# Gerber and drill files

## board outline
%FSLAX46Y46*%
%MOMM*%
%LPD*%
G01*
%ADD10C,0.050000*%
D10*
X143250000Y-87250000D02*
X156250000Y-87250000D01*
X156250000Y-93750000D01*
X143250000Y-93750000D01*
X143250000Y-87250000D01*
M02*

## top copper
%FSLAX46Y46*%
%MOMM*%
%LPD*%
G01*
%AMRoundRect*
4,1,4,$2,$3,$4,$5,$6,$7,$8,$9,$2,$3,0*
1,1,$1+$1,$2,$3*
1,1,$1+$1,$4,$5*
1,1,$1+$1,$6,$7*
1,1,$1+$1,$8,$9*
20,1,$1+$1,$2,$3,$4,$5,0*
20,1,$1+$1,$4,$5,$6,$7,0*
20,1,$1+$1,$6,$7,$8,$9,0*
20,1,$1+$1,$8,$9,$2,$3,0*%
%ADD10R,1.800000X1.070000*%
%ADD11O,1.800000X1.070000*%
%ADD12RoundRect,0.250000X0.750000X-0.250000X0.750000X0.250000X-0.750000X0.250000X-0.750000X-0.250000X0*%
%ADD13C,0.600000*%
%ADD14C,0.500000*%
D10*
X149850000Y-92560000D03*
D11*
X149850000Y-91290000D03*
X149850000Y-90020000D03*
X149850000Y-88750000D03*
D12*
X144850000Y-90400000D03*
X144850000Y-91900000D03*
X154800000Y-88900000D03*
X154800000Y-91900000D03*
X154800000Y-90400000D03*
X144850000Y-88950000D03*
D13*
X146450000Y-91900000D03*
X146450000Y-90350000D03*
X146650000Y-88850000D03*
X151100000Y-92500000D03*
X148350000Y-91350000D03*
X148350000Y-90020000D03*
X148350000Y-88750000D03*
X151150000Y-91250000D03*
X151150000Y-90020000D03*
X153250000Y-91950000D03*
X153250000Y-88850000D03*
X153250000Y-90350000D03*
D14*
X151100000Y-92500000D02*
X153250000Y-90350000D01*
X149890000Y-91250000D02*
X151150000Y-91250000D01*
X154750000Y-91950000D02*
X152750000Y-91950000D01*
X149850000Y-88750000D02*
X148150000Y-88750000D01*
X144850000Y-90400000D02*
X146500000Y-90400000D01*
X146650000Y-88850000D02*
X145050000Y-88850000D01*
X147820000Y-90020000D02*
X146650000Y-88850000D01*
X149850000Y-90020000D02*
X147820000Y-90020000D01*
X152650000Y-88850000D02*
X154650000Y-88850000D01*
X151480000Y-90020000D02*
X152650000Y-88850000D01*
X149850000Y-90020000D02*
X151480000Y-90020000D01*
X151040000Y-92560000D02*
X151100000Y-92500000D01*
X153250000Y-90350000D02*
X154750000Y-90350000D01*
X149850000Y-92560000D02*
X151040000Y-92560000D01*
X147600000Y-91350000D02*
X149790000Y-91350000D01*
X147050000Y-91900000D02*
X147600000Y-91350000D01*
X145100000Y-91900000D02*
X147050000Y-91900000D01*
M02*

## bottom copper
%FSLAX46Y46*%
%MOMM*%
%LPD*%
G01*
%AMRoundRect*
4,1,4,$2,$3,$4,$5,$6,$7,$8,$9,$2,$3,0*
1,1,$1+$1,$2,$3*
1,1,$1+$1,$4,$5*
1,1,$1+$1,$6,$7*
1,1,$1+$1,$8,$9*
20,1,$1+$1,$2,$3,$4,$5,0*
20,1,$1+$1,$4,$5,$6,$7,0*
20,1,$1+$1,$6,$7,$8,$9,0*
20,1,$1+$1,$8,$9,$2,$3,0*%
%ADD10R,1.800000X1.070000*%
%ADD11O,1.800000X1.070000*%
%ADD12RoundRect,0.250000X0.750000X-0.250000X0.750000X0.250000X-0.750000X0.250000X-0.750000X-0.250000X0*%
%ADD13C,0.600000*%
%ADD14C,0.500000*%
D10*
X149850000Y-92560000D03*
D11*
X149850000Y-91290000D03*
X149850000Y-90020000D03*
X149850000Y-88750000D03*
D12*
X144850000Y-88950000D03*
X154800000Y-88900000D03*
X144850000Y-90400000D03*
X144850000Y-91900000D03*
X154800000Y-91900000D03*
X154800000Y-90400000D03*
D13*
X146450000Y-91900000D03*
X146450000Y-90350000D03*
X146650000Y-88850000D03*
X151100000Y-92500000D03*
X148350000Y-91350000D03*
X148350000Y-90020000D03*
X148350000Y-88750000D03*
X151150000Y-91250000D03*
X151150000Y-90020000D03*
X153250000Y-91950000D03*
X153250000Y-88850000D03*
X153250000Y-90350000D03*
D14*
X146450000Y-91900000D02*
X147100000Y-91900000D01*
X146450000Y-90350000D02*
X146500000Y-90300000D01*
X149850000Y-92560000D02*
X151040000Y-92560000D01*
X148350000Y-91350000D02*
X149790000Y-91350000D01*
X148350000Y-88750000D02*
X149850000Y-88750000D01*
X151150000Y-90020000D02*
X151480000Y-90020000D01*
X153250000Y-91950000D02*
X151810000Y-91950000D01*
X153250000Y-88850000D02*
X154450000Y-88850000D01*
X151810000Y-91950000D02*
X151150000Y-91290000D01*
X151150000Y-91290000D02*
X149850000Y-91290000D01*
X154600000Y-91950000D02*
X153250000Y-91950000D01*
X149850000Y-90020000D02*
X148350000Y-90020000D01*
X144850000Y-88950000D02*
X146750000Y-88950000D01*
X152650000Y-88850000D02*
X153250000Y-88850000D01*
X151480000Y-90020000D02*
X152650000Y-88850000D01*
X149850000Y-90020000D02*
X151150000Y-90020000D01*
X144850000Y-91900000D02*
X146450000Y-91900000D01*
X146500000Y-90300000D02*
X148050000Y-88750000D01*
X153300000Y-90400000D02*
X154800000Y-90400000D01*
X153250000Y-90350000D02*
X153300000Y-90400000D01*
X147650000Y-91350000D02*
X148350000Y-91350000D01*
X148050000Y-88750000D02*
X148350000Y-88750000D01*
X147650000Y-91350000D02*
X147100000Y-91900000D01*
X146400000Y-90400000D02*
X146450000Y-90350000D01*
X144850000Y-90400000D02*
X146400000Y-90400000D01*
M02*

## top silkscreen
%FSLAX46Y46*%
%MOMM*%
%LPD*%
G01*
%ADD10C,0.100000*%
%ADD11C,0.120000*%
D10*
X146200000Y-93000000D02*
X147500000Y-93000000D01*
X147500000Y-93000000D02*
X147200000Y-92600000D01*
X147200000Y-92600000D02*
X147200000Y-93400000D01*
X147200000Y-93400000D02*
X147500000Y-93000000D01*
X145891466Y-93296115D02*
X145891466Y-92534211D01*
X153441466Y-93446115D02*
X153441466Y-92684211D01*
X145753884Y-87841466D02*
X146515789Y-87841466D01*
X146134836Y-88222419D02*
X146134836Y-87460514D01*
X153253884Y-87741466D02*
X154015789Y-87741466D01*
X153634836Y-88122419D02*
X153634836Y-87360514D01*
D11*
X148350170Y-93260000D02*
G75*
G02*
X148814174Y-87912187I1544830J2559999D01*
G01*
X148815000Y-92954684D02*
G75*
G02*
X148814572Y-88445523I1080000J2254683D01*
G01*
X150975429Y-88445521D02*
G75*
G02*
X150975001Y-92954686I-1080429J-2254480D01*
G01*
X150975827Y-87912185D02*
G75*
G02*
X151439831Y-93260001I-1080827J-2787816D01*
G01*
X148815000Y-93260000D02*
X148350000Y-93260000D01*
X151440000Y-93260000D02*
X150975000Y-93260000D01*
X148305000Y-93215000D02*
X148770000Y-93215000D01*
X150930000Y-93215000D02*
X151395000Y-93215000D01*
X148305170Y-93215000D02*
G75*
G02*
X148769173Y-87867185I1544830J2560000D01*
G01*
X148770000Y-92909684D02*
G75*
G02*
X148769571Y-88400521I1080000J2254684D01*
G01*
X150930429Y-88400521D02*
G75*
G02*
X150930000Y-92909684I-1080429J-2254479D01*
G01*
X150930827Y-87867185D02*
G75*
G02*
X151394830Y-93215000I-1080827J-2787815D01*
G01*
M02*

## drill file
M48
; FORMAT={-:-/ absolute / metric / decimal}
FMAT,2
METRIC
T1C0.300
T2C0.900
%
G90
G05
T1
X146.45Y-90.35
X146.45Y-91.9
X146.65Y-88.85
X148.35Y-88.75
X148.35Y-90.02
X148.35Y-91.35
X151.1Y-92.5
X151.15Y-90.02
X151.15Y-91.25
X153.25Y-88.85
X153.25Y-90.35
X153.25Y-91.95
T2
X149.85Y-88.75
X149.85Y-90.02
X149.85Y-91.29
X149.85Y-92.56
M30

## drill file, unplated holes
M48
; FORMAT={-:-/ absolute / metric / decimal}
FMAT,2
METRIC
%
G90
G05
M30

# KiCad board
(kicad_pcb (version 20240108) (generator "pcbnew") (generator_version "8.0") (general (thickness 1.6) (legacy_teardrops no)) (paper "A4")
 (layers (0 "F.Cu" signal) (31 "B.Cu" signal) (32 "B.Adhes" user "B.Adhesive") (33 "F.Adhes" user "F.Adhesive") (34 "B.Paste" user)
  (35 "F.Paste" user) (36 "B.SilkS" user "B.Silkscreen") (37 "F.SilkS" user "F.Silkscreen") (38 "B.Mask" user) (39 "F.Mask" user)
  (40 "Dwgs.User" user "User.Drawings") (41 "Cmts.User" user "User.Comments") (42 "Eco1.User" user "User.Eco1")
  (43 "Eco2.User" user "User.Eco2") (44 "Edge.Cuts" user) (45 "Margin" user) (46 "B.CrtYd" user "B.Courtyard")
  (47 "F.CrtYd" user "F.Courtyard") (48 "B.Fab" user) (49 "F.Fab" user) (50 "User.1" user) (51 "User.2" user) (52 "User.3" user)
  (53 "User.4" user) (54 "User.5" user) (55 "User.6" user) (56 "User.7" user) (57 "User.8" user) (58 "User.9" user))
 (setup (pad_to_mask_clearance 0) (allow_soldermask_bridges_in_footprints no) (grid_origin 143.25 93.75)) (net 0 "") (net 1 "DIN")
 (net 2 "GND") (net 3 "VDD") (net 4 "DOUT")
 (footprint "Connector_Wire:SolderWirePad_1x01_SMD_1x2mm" (layer "F.Cu") (at 144.85 90.4 90)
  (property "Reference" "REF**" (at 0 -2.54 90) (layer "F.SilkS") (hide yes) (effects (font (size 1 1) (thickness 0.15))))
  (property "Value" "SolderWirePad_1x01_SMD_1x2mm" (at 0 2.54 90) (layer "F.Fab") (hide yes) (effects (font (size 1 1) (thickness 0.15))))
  (pad "1" smd roundrect (at 0 0 90) (size 1 2) (layers "F.Cu" "F.Paste" "F.Mask") (roundrect_rratio 0.25) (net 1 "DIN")))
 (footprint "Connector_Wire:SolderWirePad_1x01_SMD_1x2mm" (layer "F.Cu") (at 144.85 91.9 90)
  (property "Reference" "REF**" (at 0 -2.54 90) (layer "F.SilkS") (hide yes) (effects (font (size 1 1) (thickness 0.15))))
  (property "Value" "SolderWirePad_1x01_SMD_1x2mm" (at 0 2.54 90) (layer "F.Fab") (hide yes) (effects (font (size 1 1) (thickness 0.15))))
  (pad "1" smd roundrect (at 0 0 90) (size 1 2) (layers "F.Cu" "F.Paste" "F.Mask") (roundrect_rratio 0.25) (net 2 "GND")))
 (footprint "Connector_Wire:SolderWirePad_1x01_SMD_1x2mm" (layer "F.Cu") (at 154.8 88.9 90)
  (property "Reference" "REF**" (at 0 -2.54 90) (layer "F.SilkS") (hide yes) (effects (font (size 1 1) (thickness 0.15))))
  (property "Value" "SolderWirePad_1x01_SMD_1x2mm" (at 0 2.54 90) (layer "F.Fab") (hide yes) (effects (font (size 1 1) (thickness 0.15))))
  (pad "1" smd roundrect (at 0 0 90) (size 1 2) (layers "F.Cu" "F.Paste" "F.Mask") (roundrect_rratio 0.25) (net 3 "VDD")))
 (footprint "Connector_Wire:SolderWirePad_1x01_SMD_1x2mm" (layer "F.Cu") (at 154.8 91.9 90)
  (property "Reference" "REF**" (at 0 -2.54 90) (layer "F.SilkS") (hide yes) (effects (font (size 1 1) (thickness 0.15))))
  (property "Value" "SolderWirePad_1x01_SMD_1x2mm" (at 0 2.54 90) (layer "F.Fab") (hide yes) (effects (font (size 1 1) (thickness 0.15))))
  (pad "1" smd roundrect (at 0 0 90) (size 1 2) (layers "F.Cu" "F.Paste" "F.Mask") (roundrect_rratio 0.25) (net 2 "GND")))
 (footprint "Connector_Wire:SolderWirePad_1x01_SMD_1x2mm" (layer "F.Cu") (at 154.8 90.4 90)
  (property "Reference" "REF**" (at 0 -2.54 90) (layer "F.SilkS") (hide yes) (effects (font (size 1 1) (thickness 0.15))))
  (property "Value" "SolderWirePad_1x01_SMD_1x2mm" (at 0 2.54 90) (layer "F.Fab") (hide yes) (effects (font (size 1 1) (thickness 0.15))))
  (pad "1" smd roundrect (at 0 0 90) (size 1 2) (layers "F.Cu" "F.Paste" "F.Mask") (roundrect_rratio 0.25) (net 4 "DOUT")))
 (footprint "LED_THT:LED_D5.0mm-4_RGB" (layer "F.Cu") (at 149.85 92.56 90)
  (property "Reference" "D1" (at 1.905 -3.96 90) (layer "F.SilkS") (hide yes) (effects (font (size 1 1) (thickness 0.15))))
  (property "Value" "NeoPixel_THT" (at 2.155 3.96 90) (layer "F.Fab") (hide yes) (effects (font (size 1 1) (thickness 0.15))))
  (fp_line (start -0.655 -1.545) (end -0.655 -1.08) (stroke (width 0.12) (type solid)) (layer "F.SilkS"))
  (fp_line (start -0.7 -1.035) (end -0.7 -1.5) (stroke (width 0.12) (type solid)) (layer "F.SilkS"))
  (fp_line (start -0.655 1.08) (end -0.655 1.545) (stroke (width 0.12) (type solid)) (layer "F.SilkS"))
  (fp_line (start -0.7 1.59) (end -0.7 1.125) (stroke (width 0.12) (type solid)) (layer "F.SilkS"))
  (fp_arc (start -0.655 -1.54483) (mid 2.163456 -2.978809) (end 4.692815 -1.080827) (stroke (width 0.12) (type solid)) (layer "F.SilkS"))
  (fp_arc (start -0.7 -1.49983) (mid 2.118456 -2.933808) (end 4.647815 -1.035827) (stroke (width 0.12) (type solid)) (layer "F.SilkS"))
  (fp_arc (start -0.349684 -1.08) (mid 1.904762 -2.5) (end 4.159479 -1.080429) (stroke (width 0.12) (type solid)) (layer "F.SilkS"))
  (fp_arc (start -0.394684 -1.035) (mid 1.859762 -2.454999) (end 4.114479 -1.035429) (stroke (width 0.12) (type solid)) (layer "F.SilkS"))
  (fp_arc (start 4.159479 1.080429) (mid 1.904762 2.5) (end -0.349684 1.08) (stroke (width 0.12) (type solid)) (layer "F.SilkS"))
  (fp_arc (start 4.692815 1.080827) (mid 2.163456 2.978808) (end -0.655 1.54483) (stroke (width 0.12) (type solid)) (layer "F.SilkS"))
  (fp_arc (start 4.114479 1.125429) (mid 1.859762 2.545001) (end -0.394684 1.125) (stroke (width 0.12) (type solid)) (layer "F.SilkS"))
  (fp_arc (start 4.647815 1.125827) (mid 2.118456 3.023809) (end -0.7 1.58983) (stroke (width 0.12) (type solid)) (layer "F.SilkS"))
  (pad "1" thru_hole rect (at 0 0 90) (size 1.07 1.8) (drill 0.9) (layers "*.Cu" "*.Mask") (remove_unused_layers no) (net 4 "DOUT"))
  (pad "2" thru_hole oval (at 1.27 0 90) (size 1.07 1.8) (drill 0.9) (layers "*.Cu" "*.Mask") (remove_unused_layers no) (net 2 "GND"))
  (pad "3" thru_hole oval (at 2.54 0 90) (size 1.07 1.8) (drill 0.9) (layers "*.Cu" "*.Mask") (remove_unused_layers no) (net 3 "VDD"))
  (pad "4" thru_hole oval (at 3.81 0 90) (size 1.07 1.8) (drill 0.9) (layers "*.Cu" "*.Mask") (remove_unused_layers no) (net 1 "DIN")))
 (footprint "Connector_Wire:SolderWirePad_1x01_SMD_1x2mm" (layer "F.Cu") (at 144.85 88.95 90)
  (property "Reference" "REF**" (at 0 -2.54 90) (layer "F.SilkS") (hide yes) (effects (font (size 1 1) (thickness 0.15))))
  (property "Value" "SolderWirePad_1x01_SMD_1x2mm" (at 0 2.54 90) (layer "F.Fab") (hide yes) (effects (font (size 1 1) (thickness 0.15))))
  (pad "1" smd roundrect (at 0 0 90) (size 1 2) (layers "F.Cu" "F.Paste" "F.Mask") (roundrect_rratio 0.25) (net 3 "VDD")))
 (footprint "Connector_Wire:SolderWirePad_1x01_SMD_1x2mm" (layer "B.Cu") (at 154.8 90.4 90)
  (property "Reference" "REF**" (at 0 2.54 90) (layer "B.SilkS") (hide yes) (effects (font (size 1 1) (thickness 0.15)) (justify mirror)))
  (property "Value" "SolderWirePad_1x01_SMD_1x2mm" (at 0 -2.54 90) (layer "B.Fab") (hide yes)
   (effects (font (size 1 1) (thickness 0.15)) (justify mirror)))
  (pad "1" smd roundrect (at 0 0 90) (size 1 2) (layers "B.Cu" "B.Paste" "B.Mask") (roundrect_rratio 0.25) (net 4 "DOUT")))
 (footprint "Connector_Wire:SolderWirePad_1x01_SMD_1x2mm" (layer "B.Cu") (at 144.85 88.95 90)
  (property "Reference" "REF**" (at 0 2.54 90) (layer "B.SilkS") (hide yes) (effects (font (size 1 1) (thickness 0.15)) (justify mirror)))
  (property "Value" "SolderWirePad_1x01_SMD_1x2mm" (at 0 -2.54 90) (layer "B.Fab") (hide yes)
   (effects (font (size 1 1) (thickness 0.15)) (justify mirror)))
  (pad "1" smd roundrect (at 0 0 90) (size 1 2) (layers "B.Cu" "B.Paste" "B.Mask") (roundrect_rratio 0.25) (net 3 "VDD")))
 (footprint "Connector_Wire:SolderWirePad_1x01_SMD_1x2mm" (layer "B.Cu") (at 154.8 88.9 90)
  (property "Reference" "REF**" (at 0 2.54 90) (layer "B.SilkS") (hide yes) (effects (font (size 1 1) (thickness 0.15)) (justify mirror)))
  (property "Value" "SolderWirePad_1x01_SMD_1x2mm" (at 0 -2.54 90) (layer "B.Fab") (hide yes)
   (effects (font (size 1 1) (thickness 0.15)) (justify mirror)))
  (pad "1" smd roundrect (at 0 0 90) (size 1 2) (layers "B.Cu" "B.Paste" "B.Mask") (roundrect_rratio 0.25) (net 3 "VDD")))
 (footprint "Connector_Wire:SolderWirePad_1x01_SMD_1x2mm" (layer "B.Cu") (at 144.85 90.4 90)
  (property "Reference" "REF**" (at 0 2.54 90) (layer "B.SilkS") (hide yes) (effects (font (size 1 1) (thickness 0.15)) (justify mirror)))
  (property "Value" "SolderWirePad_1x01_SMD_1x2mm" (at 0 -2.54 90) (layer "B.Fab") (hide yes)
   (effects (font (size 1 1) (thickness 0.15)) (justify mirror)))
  (pad "1" smd roundrect (at 0 0 90) (size 1 2) (layers "B.Cu" "B.Paste" "B.Mask") (roundrect_rratio 0.25) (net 1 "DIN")))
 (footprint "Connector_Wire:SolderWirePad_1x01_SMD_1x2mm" (layer "B.Cu") (at 144.85 91.9 90)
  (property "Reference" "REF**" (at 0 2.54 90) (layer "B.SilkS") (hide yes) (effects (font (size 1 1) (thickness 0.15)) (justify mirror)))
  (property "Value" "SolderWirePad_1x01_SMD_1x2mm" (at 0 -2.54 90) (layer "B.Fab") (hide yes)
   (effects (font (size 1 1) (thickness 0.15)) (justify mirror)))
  (pad "1" smd roundrect (at 0 0 90) (size 1 2) (layers "B.Cu" "B.Paste" "B.Mask") (roundrect_rratio 0.25) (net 2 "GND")))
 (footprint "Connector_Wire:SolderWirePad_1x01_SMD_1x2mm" (layer "B.Cu") (at 154.8 91.9 90)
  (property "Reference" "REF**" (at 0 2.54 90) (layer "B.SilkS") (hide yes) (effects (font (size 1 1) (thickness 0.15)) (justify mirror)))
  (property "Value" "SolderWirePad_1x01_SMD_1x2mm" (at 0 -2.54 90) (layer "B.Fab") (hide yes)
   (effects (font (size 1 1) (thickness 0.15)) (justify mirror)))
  (pad "1" smd roundrect (at 0 0 90) (size 1 2) (layers "B.Cu" "B.Paste" "B.Mask") (roundrect_rratio 0.25) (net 2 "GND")))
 (gr_line (start 146.2 93) (end 147.5 93) (stroke (width 0.1) (type default)) (layer "F.SilkS"))
 (gr_line (start 147.5 93) (end 147.2 92.6) (stroke (width 0.1) (type default)) (layer "F.SilkS"))
 (gr_line (start 147.2 92.6) (end 147.2 93.4) (stroke (width 0.1) (type default)) (layer "F.SilkS"))
 (gr_line (start 147.2 93.4) (end 147.5 93) (stroke (width 0.1) (type default)) (layer "F.SilkS"))
 (gr_rect (start 143.25 87.25) (end 156.25 93.75) (stroke (width 0.05) (type default)) (fill none) (layer "Edge.Cuts"))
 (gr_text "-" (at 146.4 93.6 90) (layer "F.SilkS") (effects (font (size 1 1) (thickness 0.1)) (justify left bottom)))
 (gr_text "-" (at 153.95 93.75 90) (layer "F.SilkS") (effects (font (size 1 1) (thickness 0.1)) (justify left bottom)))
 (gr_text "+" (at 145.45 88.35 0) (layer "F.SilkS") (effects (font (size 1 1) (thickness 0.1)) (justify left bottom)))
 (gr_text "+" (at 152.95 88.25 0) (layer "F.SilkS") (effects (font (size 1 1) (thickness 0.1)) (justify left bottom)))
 (segment (start 145.1 91.9) (end 147.05 91.9) (width 0.5) (layer "F.Cu") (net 2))
 (segment (start 149.89 91.25) (end 151.15 91.25) (width 0.5) (layer "F.Cu") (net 2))
 (segment (start 147.6 91.35) (end 149.79 91.35) (width 0.5) (layer "F.Cu") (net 2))
 (segment (start 154.75 91.95) (end 152.75 91.95) (width 0.5) (layer "F.Cu") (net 2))
 (segment (start 147.05 91.9) (end 147.6 91.35) (width 0.5) (layer "F.Cu") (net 2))
 (via (at 148.35 91.35) (size 0.6) (drill 0.3) (layers "F.Cu" "B.Cu") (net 2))
 (via (at 151.15 91.25) (size 0.6) (drill 0.3) (layers "F.Cu" "B.Cu") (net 2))
 (via (at 146.45 91.9) (size 0.6) (drill 0.3) (layers "F.Cu" "B.Cu") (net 2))
 (via (at 153.25 91.95) (size 0.6) (drill 0.3) (layers "F.Cu" "B.Cu") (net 2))
 (segment (start 147.65 91.35) (end 147.1 91.9) (width 0.5) (layer "B.Cu") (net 2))
 (segment (start 151.15 91.29) (end 149.85 91.29) (width 0.5) (layer "B.Cu") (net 2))
 (segment (start 153.25 91.95) (end 151.81 91.95) (width 0.5) (layer "B.Cu") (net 2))
 (segment (start 147.65 91.35) (end 148.35 91.35) (width 0.5) (layer "B.Cu") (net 2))
 (segment (start 151.81 91.95) (end 151.15 91.29) (width 0.5) (layer "B.Cu") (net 2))
 (segment (start 154.6 91.95) (end 153.25 91.95) (width 0.5) (layer "B.Cu") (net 2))
 (segment (start 144.85 91.9) (end 146.45 91.9) (width 0.5) (layer "B.Cu") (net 2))
 (segment (start 148.35 91.35) (end 149.79 91.35) (width 0.5) (layer "B.Cu") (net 2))
 (segment (start 146.45 91.9) (end 147.1 91.9) (width 0.5) (layer "B.Cu") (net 2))
 (segment (start 144.85 90.4) (end 146.5 90.4) (width 0.5) (layer "F.Cu") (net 1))
 (segment (start 149.85 88.75) (end 148.15 88.75) (width 0.5) (layer "F.Cu") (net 1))
 (via (at 148.35 88.75) (size 0.6) (drill 0.3) (layers "F.Cu" "B.Cu") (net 1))
 (via (at 146.45 90.35) (size 0.6) (drill 0.3) (layers "F.Cu" "B.Cu") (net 1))
 (segment (start 148.05 88.75) (end 148.35 88.75) (width 0.5) (layer "B.Cu") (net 1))
 (segment (start 146.45 90.35) (end 146.5 90.3) (width 0.5) (layer "B.Cu") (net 1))
 (segment (start 146.5 90.3) (end 148.05 88.75) (width 0.5) (layer "B.Cu") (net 1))
 (segment (start 146.4 90.4) (end 146.45 90.35) (width 0.5) (layer "B.Cu") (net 1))
 (segment (start 148.35 88.75) (end 149.85 88.75) (width 0.5) (layer "B.Cu") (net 1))
 (segment (start 144.85 90.4) (end 146.4 90.4) (width 0.5) (layer "B.Cu") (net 1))
 (segment (start 151.04 92.56) (end 151.1 92.5) (width 0.5) (layer "F.Cu") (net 4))
 (segment (start 153.25 90.35) (end 154.75 90.35) (width 0.5) (layer "F.Cu") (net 4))
 (segment (start 149.85 92.56) (end 151.04 92.56) (width 0.5) (layer "F.Cu") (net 4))
 (segment (start 151.1 92.5) (end 153.25 90.35) (width 0.5) (layer "F.Cu") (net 4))
 (via (at 153.25 90.35) (size 0.6) (drill 0.3) (layers "F.Cu" "B.Cu") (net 4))
 (via (at 151.1 92.5) (size 0.6) (drill 0.3) (layers "F.Cu" "B.Cu") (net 4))
 (segment (start 153.25 90.35) (end 153.3 90.4) (width 0.5) (layer "B.Cu") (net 4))
 (segment (start 153.3 90.4) (end 154.8 90.4) (width 0.5) (layer "B.Cu") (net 4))
 (segment (start 149.85 92.56) (end 151.04 92.56) (width 0.5) (layer "B.Cu") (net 4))
 (segment (start 149.85 90.02) (end 147.82 90.02) (width 0.5) (layer "F.Cu") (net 3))
 (segment (start 147.82 90.02) (end 146.65 88.85) (width 0.5) (layer "F.Cu") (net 3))
 (segment (start 146.65 88.85) (end 145.05 88.85) (width 0.5) (layer "F.Cu") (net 3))
 (segment (start 152.65 88.85) (end 154.65 88.85) (width 0.5) (layer "F.Cu") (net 3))
 (segment (start 149.85 90.02) (end 151.48 90.02) (width 0.5) (layer "F.Cu") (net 3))
 (segment (start 151.48 90.02) (end 152.65 88.85) (width 0.5) (layer "F.Cu") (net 3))
 (via (at 148.35 90.02) (size 0.6) (drill 0.3) (layers "F.Cu" "B.Cu") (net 3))
 (via (at 151.15 90.02) (size 0.6) (drill 0.3) (layers "F.Cu" "B.Cu") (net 3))
 (via (at 146.65 88.85) (size 0.6) (drill 0.3) (layers "F.Cu" "B.Cu") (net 3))
 (via (at 153.25 88.85) (size 0.6) (drill 0.3) (layers "F.Cu" "B.Cu") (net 3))
 (segment (start 144.85 88.95) (end 146.75 88.95) (width 0.5) (layer "B.Cu") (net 3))
 (segment (start 149.85 90.02) (end 151.15 90.02) (width 0.5) (layer "B.Cu") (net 3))
 (segment (start 153.25 88.85) (end 154.45 88.85) (width 0.5) (layer "B.Cu") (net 3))
 (segment (start 151.48 90.02) (end 152.65 88.85) (width 0.5) (layer "B.Cu") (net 3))
 (segment (start 152.65 88.85) (end 153.25 88.85) (width 0.5) (layer "B.Cu") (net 3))
 (segment (start 151.15 90.02) (end 151.48 90.02) (width 0.5) (layer "B.Cu") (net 3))
 (segment (start 149.85 90.02) (end 148.35 90.02) (width 0.5) (layer "B.Cu") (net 3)))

